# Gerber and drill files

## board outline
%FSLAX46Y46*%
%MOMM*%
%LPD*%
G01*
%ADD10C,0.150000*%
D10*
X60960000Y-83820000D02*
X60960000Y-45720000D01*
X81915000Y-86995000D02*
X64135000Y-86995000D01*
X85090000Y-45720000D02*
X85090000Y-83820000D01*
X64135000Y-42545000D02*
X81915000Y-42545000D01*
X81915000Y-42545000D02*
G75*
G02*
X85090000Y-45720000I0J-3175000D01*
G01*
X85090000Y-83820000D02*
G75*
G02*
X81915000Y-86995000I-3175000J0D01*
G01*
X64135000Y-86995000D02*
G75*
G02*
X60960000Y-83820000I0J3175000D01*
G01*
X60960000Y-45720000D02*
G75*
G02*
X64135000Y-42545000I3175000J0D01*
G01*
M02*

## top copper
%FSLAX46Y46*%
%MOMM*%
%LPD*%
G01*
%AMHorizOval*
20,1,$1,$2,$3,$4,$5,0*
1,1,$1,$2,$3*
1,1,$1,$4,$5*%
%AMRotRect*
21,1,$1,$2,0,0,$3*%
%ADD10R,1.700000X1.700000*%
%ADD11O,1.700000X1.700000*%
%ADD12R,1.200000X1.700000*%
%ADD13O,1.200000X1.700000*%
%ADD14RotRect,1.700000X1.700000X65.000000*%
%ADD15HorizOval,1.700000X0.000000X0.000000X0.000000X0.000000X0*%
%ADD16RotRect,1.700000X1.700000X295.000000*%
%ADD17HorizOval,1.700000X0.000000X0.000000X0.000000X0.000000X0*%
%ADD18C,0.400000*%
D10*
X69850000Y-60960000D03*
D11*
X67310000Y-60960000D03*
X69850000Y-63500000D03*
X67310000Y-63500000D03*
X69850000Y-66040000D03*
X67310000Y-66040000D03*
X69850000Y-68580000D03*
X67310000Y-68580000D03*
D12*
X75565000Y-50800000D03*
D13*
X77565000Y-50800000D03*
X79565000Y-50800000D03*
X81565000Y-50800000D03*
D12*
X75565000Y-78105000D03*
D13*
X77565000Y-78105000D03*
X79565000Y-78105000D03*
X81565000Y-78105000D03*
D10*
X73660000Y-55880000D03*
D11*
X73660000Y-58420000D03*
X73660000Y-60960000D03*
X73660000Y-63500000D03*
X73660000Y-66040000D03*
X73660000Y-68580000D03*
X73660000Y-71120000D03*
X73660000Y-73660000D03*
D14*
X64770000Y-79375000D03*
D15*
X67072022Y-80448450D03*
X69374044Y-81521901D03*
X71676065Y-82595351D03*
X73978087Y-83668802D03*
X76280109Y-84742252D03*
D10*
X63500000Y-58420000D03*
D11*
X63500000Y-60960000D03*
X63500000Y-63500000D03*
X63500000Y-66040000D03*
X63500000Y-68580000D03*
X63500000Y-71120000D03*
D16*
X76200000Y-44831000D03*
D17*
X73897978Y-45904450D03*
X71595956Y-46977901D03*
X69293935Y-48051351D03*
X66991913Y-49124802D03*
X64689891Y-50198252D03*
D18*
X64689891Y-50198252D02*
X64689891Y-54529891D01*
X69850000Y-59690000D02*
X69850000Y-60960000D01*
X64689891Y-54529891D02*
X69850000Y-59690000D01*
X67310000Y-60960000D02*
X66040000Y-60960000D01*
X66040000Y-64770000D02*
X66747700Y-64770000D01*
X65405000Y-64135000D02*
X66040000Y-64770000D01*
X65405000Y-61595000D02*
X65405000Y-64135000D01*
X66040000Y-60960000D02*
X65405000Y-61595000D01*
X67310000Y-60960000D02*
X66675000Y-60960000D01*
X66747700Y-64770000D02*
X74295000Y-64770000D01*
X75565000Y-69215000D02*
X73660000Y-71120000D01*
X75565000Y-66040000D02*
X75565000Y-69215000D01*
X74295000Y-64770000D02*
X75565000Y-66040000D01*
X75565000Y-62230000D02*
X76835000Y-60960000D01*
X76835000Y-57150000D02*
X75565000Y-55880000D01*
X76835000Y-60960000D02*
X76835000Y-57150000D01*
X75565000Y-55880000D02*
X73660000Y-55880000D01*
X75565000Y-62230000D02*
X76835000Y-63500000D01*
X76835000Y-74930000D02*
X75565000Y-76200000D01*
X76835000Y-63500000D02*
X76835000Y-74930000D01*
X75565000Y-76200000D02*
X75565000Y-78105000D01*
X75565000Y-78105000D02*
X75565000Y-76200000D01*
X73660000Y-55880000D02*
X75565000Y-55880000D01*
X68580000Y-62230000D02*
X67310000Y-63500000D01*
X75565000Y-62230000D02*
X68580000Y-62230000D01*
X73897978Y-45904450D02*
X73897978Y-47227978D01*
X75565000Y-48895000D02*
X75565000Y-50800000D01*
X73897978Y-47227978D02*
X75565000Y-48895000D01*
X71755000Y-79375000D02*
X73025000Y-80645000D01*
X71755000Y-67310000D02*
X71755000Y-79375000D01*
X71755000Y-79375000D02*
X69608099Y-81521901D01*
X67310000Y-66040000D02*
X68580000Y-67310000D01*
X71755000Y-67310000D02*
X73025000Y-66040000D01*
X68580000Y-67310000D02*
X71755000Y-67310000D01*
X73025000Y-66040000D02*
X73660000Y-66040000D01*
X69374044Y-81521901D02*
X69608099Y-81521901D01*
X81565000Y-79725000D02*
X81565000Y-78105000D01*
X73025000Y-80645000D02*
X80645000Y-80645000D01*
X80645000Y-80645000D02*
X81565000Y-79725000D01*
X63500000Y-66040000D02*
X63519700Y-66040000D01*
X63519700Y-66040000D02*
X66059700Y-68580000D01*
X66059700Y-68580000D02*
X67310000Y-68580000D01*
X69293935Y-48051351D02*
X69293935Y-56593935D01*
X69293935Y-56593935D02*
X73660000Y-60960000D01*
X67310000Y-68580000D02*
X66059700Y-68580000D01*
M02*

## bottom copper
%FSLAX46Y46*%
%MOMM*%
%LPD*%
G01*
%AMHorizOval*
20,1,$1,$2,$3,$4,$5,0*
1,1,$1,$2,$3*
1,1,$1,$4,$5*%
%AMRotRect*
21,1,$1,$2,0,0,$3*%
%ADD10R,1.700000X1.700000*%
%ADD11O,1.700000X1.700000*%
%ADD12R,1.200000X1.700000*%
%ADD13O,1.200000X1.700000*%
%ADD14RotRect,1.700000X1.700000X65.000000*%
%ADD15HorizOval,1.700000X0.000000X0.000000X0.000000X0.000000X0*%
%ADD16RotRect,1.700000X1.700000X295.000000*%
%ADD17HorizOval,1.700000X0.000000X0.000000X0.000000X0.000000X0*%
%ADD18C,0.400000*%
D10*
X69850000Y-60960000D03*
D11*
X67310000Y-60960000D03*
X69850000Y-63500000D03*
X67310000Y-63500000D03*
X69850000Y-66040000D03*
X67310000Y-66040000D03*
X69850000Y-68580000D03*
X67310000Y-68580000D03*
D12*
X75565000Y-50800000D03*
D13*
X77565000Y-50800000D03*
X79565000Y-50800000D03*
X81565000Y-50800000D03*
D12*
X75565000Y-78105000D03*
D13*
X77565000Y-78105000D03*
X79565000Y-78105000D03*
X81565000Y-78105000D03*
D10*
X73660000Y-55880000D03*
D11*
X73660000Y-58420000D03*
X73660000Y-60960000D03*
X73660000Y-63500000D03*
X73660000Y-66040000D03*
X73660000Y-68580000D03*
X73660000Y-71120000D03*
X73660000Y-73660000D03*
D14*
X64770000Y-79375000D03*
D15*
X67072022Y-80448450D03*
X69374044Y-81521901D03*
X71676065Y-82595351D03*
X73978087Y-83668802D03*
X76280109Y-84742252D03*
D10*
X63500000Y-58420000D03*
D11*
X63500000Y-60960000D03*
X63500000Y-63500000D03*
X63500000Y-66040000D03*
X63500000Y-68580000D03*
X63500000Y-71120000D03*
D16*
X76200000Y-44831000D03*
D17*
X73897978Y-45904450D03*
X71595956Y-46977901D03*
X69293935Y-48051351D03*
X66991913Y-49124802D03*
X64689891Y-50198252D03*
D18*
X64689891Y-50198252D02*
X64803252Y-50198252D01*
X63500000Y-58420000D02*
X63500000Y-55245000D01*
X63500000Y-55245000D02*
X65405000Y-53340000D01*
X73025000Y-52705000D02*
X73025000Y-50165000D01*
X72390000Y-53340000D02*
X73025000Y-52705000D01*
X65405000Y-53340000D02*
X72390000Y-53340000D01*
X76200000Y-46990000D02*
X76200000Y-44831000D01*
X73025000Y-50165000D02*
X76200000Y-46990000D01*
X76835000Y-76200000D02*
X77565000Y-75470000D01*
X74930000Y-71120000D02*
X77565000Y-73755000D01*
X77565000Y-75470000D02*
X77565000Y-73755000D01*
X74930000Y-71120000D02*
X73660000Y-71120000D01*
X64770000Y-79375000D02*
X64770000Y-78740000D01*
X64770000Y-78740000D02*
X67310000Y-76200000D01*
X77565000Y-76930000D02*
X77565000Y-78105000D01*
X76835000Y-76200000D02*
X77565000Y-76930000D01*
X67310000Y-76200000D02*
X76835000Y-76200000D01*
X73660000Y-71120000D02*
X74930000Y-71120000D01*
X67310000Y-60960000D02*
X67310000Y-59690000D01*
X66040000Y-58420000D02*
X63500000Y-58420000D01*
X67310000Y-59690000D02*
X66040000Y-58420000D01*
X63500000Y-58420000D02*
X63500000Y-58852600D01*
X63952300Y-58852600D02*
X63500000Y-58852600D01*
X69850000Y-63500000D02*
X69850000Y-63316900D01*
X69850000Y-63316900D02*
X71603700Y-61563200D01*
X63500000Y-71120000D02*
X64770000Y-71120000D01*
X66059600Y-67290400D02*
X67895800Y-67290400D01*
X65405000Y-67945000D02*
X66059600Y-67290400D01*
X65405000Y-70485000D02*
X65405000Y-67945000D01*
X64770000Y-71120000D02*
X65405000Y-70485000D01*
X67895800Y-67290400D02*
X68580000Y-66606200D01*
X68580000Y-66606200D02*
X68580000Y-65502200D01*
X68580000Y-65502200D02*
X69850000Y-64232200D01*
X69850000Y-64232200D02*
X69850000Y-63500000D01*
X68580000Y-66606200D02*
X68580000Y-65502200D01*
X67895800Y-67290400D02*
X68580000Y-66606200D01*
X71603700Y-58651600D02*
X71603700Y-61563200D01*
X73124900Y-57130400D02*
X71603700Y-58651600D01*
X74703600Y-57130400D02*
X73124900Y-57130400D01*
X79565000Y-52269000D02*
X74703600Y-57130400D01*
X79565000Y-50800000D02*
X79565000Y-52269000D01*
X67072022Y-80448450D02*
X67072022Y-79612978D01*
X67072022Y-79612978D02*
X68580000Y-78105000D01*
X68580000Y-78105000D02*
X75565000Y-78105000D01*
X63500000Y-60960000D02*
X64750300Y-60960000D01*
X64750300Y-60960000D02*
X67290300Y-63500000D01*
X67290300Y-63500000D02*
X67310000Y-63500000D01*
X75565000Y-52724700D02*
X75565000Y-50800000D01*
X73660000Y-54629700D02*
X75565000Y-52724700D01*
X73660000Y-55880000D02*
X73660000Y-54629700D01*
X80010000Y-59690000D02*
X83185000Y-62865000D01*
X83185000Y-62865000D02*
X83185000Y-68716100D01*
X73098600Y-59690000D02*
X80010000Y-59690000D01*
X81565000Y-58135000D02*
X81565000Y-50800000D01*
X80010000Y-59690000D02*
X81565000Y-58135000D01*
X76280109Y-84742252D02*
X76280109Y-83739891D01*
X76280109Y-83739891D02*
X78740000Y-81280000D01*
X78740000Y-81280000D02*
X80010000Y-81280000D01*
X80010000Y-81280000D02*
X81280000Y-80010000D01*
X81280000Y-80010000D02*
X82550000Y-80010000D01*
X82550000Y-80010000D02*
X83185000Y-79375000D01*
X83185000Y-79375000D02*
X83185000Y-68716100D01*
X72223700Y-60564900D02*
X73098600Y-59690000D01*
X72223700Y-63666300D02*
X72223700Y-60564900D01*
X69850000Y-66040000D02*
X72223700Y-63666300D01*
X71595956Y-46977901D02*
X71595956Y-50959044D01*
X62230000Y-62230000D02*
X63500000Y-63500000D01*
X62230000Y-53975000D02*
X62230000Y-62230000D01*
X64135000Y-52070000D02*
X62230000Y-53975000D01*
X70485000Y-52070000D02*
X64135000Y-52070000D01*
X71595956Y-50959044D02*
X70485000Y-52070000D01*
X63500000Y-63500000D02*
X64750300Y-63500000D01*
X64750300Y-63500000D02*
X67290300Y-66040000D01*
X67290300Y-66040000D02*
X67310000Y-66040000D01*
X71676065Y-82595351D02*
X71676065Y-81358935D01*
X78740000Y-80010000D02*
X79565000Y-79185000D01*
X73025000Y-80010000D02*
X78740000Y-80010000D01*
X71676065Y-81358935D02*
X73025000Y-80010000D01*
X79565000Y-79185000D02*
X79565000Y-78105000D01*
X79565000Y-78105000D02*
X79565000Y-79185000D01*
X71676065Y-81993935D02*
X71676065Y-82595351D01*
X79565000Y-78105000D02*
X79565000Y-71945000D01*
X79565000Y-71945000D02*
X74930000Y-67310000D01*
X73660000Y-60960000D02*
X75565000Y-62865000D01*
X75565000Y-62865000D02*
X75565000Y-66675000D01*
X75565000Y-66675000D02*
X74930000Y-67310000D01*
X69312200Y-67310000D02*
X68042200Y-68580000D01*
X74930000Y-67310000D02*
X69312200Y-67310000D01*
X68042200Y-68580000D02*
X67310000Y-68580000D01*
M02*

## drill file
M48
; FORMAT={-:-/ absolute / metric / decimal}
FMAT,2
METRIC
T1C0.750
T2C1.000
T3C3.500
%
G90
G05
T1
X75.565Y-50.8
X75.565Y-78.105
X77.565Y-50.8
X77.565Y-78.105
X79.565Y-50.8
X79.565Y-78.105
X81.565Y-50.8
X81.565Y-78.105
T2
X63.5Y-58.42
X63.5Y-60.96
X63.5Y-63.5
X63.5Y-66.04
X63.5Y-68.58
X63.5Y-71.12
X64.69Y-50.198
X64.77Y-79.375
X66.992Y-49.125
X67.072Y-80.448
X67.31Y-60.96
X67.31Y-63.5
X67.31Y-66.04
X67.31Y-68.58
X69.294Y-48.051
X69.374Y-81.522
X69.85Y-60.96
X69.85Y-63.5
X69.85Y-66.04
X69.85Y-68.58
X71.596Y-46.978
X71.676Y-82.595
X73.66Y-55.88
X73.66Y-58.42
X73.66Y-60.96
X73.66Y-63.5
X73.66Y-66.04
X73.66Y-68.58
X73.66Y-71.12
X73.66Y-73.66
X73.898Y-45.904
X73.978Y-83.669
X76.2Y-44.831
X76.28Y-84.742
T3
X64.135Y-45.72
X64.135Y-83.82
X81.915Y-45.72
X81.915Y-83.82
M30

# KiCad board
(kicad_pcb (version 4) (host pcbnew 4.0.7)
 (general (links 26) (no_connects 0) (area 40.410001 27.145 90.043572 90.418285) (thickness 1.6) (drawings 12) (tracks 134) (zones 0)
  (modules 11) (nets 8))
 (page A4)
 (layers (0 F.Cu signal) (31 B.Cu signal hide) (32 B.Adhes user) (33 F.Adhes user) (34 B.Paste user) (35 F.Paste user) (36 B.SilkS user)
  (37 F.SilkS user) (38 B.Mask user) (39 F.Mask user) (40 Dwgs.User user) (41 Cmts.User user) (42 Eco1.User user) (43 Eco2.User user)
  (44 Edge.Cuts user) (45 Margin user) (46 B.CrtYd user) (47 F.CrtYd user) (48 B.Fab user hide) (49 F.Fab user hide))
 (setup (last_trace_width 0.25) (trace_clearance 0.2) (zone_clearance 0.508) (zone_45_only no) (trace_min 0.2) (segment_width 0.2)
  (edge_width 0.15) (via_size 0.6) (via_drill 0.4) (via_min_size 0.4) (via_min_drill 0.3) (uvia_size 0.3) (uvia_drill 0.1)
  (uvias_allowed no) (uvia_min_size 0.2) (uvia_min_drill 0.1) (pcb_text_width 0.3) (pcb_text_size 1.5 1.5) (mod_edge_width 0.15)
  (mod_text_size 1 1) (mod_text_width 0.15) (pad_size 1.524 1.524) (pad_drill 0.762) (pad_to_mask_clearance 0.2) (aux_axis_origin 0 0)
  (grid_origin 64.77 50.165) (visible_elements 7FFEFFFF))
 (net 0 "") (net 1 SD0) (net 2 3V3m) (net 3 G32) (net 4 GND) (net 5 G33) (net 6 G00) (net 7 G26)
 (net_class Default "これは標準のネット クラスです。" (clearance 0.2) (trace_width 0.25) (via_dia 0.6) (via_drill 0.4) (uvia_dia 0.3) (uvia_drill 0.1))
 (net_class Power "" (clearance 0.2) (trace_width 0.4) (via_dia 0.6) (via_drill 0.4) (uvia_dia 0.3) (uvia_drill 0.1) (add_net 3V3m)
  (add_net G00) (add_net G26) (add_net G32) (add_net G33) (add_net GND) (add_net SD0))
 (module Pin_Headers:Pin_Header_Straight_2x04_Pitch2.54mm (layer B.Cu) (at 69.85 60.96 180)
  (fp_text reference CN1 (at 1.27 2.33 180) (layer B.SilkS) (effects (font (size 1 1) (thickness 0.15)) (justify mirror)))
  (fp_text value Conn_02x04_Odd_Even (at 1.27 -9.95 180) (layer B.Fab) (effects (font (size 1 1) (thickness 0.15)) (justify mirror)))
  (pad 1 thru_hole rect (at 0 0 180) (size 1.7 1.7) (drill 1) (layers *.Cu *.Mask) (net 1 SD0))
  (pad 2 thru_hole oval (at 2.54 0 180) (size 1.7 1.7) (drill 1) (layers *.Cu *.Mask) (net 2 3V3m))
  (pad 3 thru_hole oval (at 0 -2.54 180) (size 1.7 1.7) (drill 1) (layers *.Cu *.Mask) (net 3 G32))
  (pad 4 thru_hole oval (at 2.54 -2.54 180) (size 1.7 1.7) (drill 1) (layers *.Cu *.Mask) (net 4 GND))
  (pad 5 thru_hole oval (at 0 -5.08 180) (size 1.7 1.7) (drill 1) (layers *.Cu *.Mask) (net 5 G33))
  (pad 6 thru_hole oval (at 2.54 -5.08 180) (size 1.7 1.7) (drill 1) (layers *.Cu *.Mask) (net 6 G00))
  (pad 7 thru_hole oval (at 0 -7.62 180) (size 1.7 1.7) (drill 1) (layers *.Cu *.Mask))
  (pad 8 thru_hole oval (at 2.54 -7.62 180) (size 1.7 1.7) (drill 1) (layers *.Cu *.Mask) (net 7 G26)))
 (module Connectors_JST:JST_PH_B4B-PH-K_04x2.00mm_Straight (layer F.Cu) (at 75.565 50.8)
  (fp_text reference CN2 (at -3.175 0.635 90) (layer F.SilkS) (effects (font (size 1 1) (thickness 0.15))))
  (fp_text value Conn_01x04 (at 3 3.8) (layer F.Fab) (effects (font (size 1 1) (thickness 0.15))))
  (pad 1 thru_hole rect (at 0 0) (size 1.2 1.7) (drill 0.75) (layers *.Cu *.Mask) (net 4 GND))
  (pad 2 thru_hole oval (at 2 0) (size 1.2 1.7) (drill 0.75) (layers *.Cu *.Mask))
  (pad 3 thru_hole oval (at 4 0) (size 1.2 1.7) (drill 0.75) (layers *.Cu *.Mask) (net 3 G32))
  (pad 4 thru_hole oval (at 6 0) (size 1.2 1.7) (drill 0.75) (layers *.Cu *.Mask) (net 5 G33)))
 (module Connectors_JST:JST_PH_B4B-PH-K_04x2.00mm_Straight (layer F.Cu) (at 75.565 78.105)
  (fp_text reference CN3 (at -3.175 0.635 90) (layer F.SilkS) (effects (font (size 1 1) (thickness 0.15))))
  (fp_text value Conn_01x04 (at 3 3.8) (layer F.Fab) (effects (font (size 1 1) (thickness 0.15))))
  (pad 1 thru_hole rect (at 0 0) (size 1.2 1.7) (drill 0.75) (layers *.Cu *.Mask) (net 4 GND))
  (pad 2 thru_hole oval (at 2 0) (size 1.2 1.7) (drill 0.75) (layers *.Cu *.Mask) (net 2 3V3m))
  (pad 3 thru_hole oval (at 4 0) (size 1.2 1.7) (drill 0.75) (layers *.Cu *.Mask) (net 7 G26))
  (pad 4 thru_hole oval (at 6 0) (size 1.2 1.7) (drill 0.75) (layers *.Cu *.Mask) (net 6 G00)))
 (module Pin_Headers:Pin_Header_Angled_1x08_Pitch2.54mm (layer F.Cu) (at 73.66 55.88)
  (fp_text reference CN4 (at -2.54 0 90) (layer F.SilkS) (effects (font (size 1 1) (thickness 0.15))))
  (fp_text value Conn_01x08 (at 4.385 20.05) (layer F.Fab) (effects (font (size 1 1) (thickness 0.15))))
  (pad 1 thru_hole rect (at 0 0) (size 1.7 1.7) (drill 1) (layers *.Cu *.Mask) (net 4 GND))
  (pad 2 thru_hole oval (at 0 2.54) (size 1.7 1.7) (drill 1) (layers *.Cu *.Mask))
  (pad 3 thru_hole oval (at 0 5.08) (size 1.7 1.7) (drill 1) (layers *.Cu *.Mask) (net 7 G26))
  (pad 4 thru_hole oval (at 0 7.62) (size 1.7 1.7) (drill 1) (layers *.Cu *.Mask))
  (pad 5 thru_hole oval (at 0 10.16) (size 1.7 1.7) (drill 1) (layers *.Cu *.Mask) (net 6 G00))
  (pad 6 thru_hole oval (at 0 12.7) (size 1.7 1.7) (drill 1) (layers *.Cu *.Mask))
  (pad 7 thru_hole oval (at 0 15.24) (size 1.7 1.7) (drill 1) (layers *.Cu *.Mask) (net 2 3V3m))
  (pad 8 thru_hole oval (at 0 17.78) (size 1.7 1.7) (drill 1) (layers *.Cu *.Mask)))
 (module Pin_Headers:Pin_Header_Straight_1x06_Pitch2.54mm (layer F.Cu) (at 64.77 79.375 65)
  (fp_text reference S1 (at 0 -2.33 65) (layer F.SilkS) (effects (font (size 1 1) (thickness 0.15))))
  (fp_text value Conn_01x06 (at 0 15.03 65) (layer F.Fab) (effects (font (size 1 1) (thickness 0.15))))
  (pad 1 thru_hole rect (at 0 0 65) (size 1.7 1.7) (drill 1) (layers *.Cu *.Mask) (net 2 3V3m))
  (pad 2 thru_hole oval (at 0 2.54 65) (size 1.7 1.7) (drill 1) (layers *.Cu *.Mask) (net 4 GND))
  (pad 3 thru_hole oval (at 0 5.08 65) (size 1.7 1.7) (drill 1) (layers *.Cu *.Mask) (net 6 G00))
  (pad 4 thru_hole oval (at 0 7.62 65) (size 1.7 1.7) (drill 1) (layers *.Cu *.Mask) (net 7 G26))
  (pad 5 thru_hole oval (at 0 10.16 65) (size 1.7 1.7) (drill 1) (layers *.Cu *.Mask))
  (pad 6 thru_hole oval (at 0 12.7 65) (size 1.7 1.7) (drill 1) (layers *.Cu *.Mask) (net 5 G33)))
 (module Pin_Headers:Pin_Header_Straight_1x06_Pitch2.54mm (layer F.Cu) (at 63.5 58.42)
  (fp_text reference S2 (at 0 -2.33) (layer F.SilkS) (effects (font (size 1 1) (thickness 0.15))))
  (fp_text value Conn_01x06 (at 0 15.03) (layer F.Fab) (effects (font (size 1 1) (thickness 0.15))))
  (pad 1 thru_hole rect (at 0 0) (size 1.7 1.7) (drill 1) (layers *.Cu *.Mask) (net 2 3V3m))
  (pad 2 thru_hole oval (at 0 2.54) (size 1.7 1.7) (drill 1) (layers *.Cu *.Mask) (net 4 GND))
  (pad 3 thru_hole oval (at 0 5.08) (size 1.7 1.7) (drill 1) (layers *.Cu *.Mask) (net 6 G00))
  (pad 4 thru_hole oval (at 0 7.62) (size 1.7 1.7) (drill 1) (layers *.Cu *.Mask) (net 7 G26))
  (pad 5 thru_hole oval (at 0 10.16) (size 1.7 1.7) (drill 1) (layers *.Cu *.Mask))
  (pad 6 thru_hole oval (at 0 12.7) (size 1.7 1.7) (drill 1) (layers *.Cu *.Mask) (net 3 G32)))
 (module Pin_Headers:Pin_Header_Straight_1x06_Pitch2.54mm (layer F.Cu) (at 76.2 44.831 295)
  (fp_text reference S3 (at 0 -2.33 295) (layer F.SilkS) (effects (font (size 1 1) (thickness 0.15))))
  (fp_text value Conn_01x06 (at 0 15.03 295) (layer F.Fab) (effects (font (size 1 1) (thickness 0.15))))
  (pad 1 thru_hole rect (at 0 0 295) (size 1.7 1.7) (drill 1) (layers *.Cu *.Mask) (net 2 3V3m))
  (pad 2 thru_hole oval (at 0 2.54 295) (size 1.7 1.7) (drill 1) (layers *.Cu *.Mask) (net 4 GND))
  (pad 3 thru_hole oval (at 0 5.08 295) (size 1.7 1.7) (drill 1) (layers *.Cu *.Mask) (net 6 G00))
  (pad 4 thru_hole oval (at 0 7.62 295) (size 1.7 1.7) (drill 1) (layers *.Cu *.Mask) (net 7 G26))
  (pad 5 thru_hole oval (at 0 10.16 295) (size 1.7 1.7) (drill 1) (layers *.Cu *.Mask))
  (pad 6 thru_hole oval (at 0 12.7 295) (size 1.7 1.7) (drill 1) (layers *.Cu *.Mask) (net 1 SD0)))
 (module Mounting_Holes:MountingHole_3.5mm (layer F.Cu) (at 64.135 45.72)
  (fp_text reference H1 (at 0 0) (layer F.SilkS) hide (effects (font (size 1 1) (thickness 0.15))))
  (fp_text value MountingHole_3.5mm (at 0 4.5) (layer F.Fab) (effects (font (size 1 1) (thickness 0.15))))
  (pad 1 np_thru_hole circle (at 0 0) (size 3.5 3.5) (drill 3.5) (layers *.Cu *.Mask)))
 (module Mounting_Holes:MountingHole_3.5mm (layer F.Cu) (at 81.915 45.72)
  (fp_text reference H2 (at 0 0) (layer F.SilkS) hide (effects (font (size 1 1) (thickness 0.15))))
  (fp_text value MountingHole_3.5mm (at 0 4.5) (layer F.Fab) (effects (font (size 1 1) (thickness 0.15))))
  (pad 1 np_thru_hole circle (at 0 0) (size 3.5 3.5) (drill 3.5) (layers *.Cu *.Mask)))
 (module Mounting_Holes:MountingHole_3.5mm (layer F.Cu) (at 64.135 83.82)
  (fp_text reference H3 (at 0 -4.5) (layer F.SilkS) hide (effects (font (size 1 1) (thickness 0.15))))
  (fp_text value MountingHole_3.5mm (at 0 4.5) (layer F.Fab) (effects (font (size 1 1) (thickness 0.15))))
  (pad 1 np_thru_hole circle (at 0 0) (size 3.5 3.5) (drill 3.5) (layers *.Cu *.Mask)))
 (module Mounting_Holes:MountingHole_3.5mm (layer F.Cu) (at 81.915 83.82)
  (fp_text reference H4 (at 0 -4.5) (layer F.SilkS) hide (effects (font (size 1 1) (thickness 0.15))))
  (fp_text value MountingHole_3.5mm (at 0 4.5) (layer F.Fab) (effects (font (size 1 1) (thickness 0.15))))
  (pad 1 np_thru_hole circle (at 0 0) (size 3.5 3.5) (drill 3.5) (layers *.Cu *.Mask)))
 (gr_line (start 60.96 83.82) (end 60.96 45.72) (angle 90) (layer Edge.Cuts) (width 0.15))
 (gr_line (start 81.915 86.995) (end 64.135 86.995) (angle 90) (layer Edge.Cuts) (width 0.15))
 (gr_line (start 85.09 45.72) (end 85.09 83.82) (angle 90) (layer Edge.Cuts) (width 0.15))
 (gr_line (start 64.135 42.545) (end 81.915 42.545) (angle 90) (layer Edge.Cuts) (width 0.15))
 (gr_arc (start 81.915 45.72) (end 81.915 42.545) (angle 90) (layer Edge.Cuts) (width 0.15))
 (gr_arc (start 81.915 83.82) (end 85.09 83.82) (angle 90) (layer Edge.Cuts) (width 0.15))
 (gr_arc (start 64.135 83.82) (end 64.135 86.995) (angle 90) (layer Edge.Cuts) (width 0.15))
 (gr_arc (start 64.135 45.72) (end 60.96 45.72) (angle 90) (layer Edge.Cuts) (width 0.15))
 (segment (start 64.689891 50.198252) (end 64.689891 54.529891) (width 0.4) (layer F.Cu) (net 1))
 (segment (start 69.85 59.69) (end 69.85 60.96) (width 0.4) (layer F.Cu) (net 1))
 (segment (start 64.689891 54.529891) (end 69.85 59.69) (width 0.4) (layer F.Cu) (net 1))
 (segment (start 64.689891 50.198252) (end 64.803252 50.198252) (width 0.4) (layer B.Cu) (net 1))
 (segment (start 63.5 58.42) (end 63.5 55.245) (width 0.4) (layer B.Cu) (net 2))
 (segment (start 63.5 55.245) (end 65.405 53.34) (width 0.4) (layer B.Cu) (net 2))
 (segment (start 73.025 52.705) (end 73.025 50.165) (width 0.4) (layer B.Cu) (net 2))
 (segment (start 72.39 53.34) (end 73.025 52.705) (width 0.4) (layer B.Cu) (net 2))
 (segment (start 65.405 53.34) (end 72.39 53.34) (width 0.4) (layer B.Cu) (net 2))
 (segment (start 76.2 46.99) (end 76.2 44.831) (width 0.4) (layer B.Cu) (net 2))
 (segment (start 73.025 50.165) (end 76.2 46.99) (width 0.4) (layer B.Cu) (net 2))
 (segment (start 67.31 60.96) (end 66.04 60.96) (width 0.4) (layer F.Cu) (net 2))
 (segment (start 66.04 64.77) (end 66.7477 64.77) (width 0.4) (layer F.Cu) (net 2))
 (segment (start 65.405 64.135) (end 66.04 64.77) (width 0.4) (layer F.Cu) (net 2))
 (segment (start 65.405 61.595) (end 65.405 64.135) (width 0.4) (layer F.Cu) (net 2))
 (segment (start 66.04 60.96) (end 65.405 61.595) (width 0.4) (layer F.Cu) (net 2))
 (segment (start 67.31 60.96) (end 66.675 60.96) (width 0.4) (layer F.Cu) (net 2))
 (segment (start 66.7477 64.77) (end 74.295 64.77) (width 0.4) (layer F.Cu) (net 2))
 (segment (start 75.565 69.215) (end 73.66 71.12) (width 0.4) (layer F.Cu) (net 2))
 (segment (start 75.565 66.04) (end 75.565 69.215) (width 0.4) (layer F.Cu) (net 2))
 (segment (start 74.295 64.77) (end 75.565 66.04) (width 0.4) (layer F.Cu) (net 2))
 (segment (start 76.835 76.2) (end 77.565 75.47) (width 0.4) (layer B.Cu) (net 2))
 (segment (start 74.93 71.12) (end 77.565 73.755) (width 0.4) (layer B.Cu) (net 2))
 (segment (start 77.565 75.47) (end 77.565 73.755) (width 0.4) (layer B.Cu) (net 2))
 (segment (start 74.93 71.12) (end 73.66 71.12) (width 0.4) (layer B.Cu) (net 2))
 (segment (start 64.77 79.375) (end 64.77 78.74) (width 0.4) (layer B.Cu) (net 2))
 (segment (start 64.77 78.74) (end 67.31 76.2) (width 0.4) (layer B.Cu) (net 2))
 (segment (start 77.565 76.93) (end 77.565 78.105) (width 0.4) (layer B.Cu) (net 2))
 (segment (start 76.835 76.2) (end 77.565 76.93) (width 0.4) (layer B.Cu) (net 2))
 (segment (start 67.31 76.2) (end 76.835 76.2) (width 0.4) (layer B.Cu) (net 2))
 (segment (start 73.66 71.12) (end 74.93 71.12) (width 0.4) (layer B.Cu) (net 2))
 (segment (start 67.31 60.96) (end 67.31 59.69) (width 0.4) (layer B.Cu) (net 2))
 (segment (start 66.04 58.42) (end 63.5 58.42) (width 0.4) (layer B.Cu) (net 2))
 (segment (start 67.31 59.69) (end 66.04 58.42) (width 0.4) (layer B.Cu) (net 2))
 (segment (start 63.5 58.42) (end 63.5 58.8526) (width 0.4) (layer B.Cu) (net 2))
 (segment (start 63.9523 58.8526) (end 63.5 58.8526) (width 0.4) (layer B.Cu) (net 2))
 (segment (start 69.85 63.5) (end 69.85 63.3169) (width 0.4) (layer B.Cu) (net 3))
 (segment (start 69.85 63.3169) (end 71.6037 61.5632) (width 0.4) (layer B.Cu) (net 3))
 (segment (start 63.5 71.12) (end 64.77 71.12) (width 0.4) (layer B.Cu) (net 3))
 (segment (start 66.0596 67.2904) (end 67.8958 67.2904) (width 0.4) (layer B.Cu) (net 3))
 (segment (start 65.405 67.945) (end 66.0596 67.2904) (width 0.4) (layer B.Cu) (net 3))
 (segment (start 65.405 70.485) (end 65.405 67.945) (width 0.4) (layer B.Cu) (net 3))
 (segment (start 64.77 71.12) (end 65.405 70.485) (width 0.4) (layer B.Cu) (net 3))
 (segment (start 67.8958 67.2904) (end 68.58 66.6062) (width 0.4) (layer B.Cu) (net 3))
 (segment (start 68.58 66.6062) (end 68.58 65.5022) (width 0.4) (layer B.Cu) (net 3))
 (segment (start 68.58 65.5022) (end 69.85 64.2322) (width 0.4) (layer B.Cu) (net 3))
 (segment (start 69.85 64.2322) (end 69.85 63.5) (width 0.4) (layer B.Cu) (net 3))
 (segment (start 68.58 66.6062) (end 68.58 65.5022) (width 0.4) (layer B.Cu) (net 3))
 (segment (start 67.8958 67.2904) (end 68.58 66.6062) (width 0.4) (layer B.Cu) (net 3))
 (segment (start 71.6037 58.6516) (end 71.6037 61.5632) (width 0.4) (layer B.Cu) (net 3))
 (segment (start 73.1249 57.1304) (end 71.6037 58.6516) (width 0.4) (layer B.Cu) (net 3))
 (segment (start 74.7036 57.1304) (end 73.1249 57.1304) (width 0.4) (layer B.Cu) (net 3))
 (segment (start 79.565 52.269) (end 74.7036 57.1304) (width 0.4) (layer B.Cu) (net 3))
 (segment (start 79.565 50.8) (end 79.565 52.269) (width 0.4) (layer B.Cu) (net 3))
 (segment (start 75.565 62.23) (end 76.835 60.96) (width 0.4) (layer F.Cu) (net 4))
 (segment (start 76.835 57.15) (end 75.565 55.88) (width 0.4) (layer F.Cu) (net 4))
 (segment (start 76.835 60.96) (end 76.835 57.15) (width 0.4) (layer F.Cu) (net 4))
 (segment (start 75.565 55.88) (end 73.66 55.88) (width 0.4) (layer F.Cu) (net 4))
 (segment (start 75.565 62.23) (end 76.835 63.5) (width 0.4) (layer F.Cu) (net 4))
 (segment (start 76.835 74.93) (end 75.565 76.2) (width 0.4) (layer F.Cu) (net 4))
 (segment (start 76.835 63.5) (end 76.835 74.93) (width 0.4) (layer F.Cu) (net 4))
 (segment (start 75.565 76.2) (end 75.565 78.105) (width 0.4) (layer F.Cu) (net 4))
 (segment (start 75.565 78.105) (end 75.565 76.2) (width 0.4) (layer F.Cu) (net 4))
 (segment (start 73.66 55.88) (end 75.565 55.88) (width 0.4) (layer F.Cu) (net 4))
 (segment (start 68.58 62.23) (end 67.31 63.5) (width 0.4) (layer F.Cu) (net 4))
 (segment (start 75.565 62.23) (end 68.58 62.23) (width 0.4) (layer F.Cu) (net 4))
 (segment (start 67.072022 80.44845) (end 67.072022 79.612978) (width 0.4) (layer B.Cu) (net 4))
 (segment (start 67.072022 79.612978) (end 68.58 78.105) (width 0.4) (layer B.Cu) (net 4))
 (segment (start 68.58 78.105) (end 75.565 78.105) (width 0.4) (layer B.Cu) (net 4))
 (segment (start 63.5 60.96) (end 64.7503 60.96) (width 0.4) (layer B.Cu) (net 4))
 (segment (start 64.7503 60.96) (end 67.2903 63.5) (width 0.4) (layer B.Cu) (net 4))
 (segment (start 67.2903 63.5) (end 67.31 63.5) (width 0.4) (layer B.Cu) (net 4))
 (segment (start 73.897978 45.90445) (end 73.897978 47.227978) (width 0.4) (layer F.Cu) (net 4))
 (segment (start 75.565 48.895) (end 75.565 50.8) (width 0.4) (layer F.Cu) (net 4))
 (segment (start 73.897978 47.227978) (end 75.565 48.895) (width 0.4) (layer F.Cu) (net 4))
 (segment (start 75.565 52.7247) (end 75.565 50.8) (width 0.4) (layer B.Cu) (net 4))
 (segment (start 73.66 54.6297) (end 75.565 52.7247) (width 0.4) (layer B.Cu) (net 4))
 (segment (start 73.66 55.88) (end 73.66 54.6297) (width 0.4) (layer B.Cu) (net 4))
 (segment (start 80.01 59.69) (end 83.185 62.865) (width 0.4) (layer B.Cu) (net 5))
 (segment (start 83.185 62.865) (end 83.185 68.7161) (width 0.4) (layer B.Cu) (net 5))
 (segment (start 73.0986 59.69) (end 80.01 59.69) (width 0.4) (layer B.Cu) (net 5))
 (segment (start 81.565 58.135) (end 81.565 50.8) (width 0.4) (layer B.Cu) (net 5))
 (segment (start 80.01 59.69) (end 81.565 58.135) (width 0.4) (layer B.Cu) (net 5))
 (segment (start 76.280109 84.742252) (end 76.280109 83.739891) (width 0.4) (layer B.Cu) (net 5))
 (segment (start 76.280109 83.739891) (end 78.74 81.28) (width 0.4) (layer B.Cu) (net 5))
 (segment (start 78.74 81.28) (end 80.01 81.28) (width 0.4) (layer B.Cu) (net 5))
 (segment (start 80.01 81.28) (end 81.28 80.01) (width 0.4) (layer B.Cu) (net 5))
 (segment (start 81.28 80.01) (end 82.55 80.01) (width 0.4) (layer B.Cu) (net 5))
 (segment (start 82.55 80.01) (end 83.185 79.375) (width 0.4) (layer B.Cu) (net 5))
 (segment (start 83.185 79.375) (end 83.185 68.7161) (width 0.4) (layer B.Cu) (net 5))
 (segment (start 72.2237 60.5649) (end 73.0986 59.69) (width 0.4) (layer B.Cu) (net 5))
 (segment (start 72.2237 63.6663) (end 72.2237 60.5649) (width 0.4) (layer B.Cu) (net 5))
 (segment (start 69.85 66.04) (end 72.2237 63.6663) (width 0.4) (layer B.Cu) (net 5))
 (segment (start 71.595956 46.977901) (end 71.595956 50.959044) (width 0.4) (layer B.Cu) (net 6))
 (segment (start 62.23 62.23) (end 63.5 63.5) (width 0.4) (layer B.Cu) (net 6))
 (segment (start 62.23 53.975) (end 62.23 62.23) (width 0.4) (layer B.Cu) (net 6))
 (segment (start 64.135 52.07) (end 62.23 53.975) (width 0.4) (layer B.Cu) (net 6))
 (segment (start 70.485 52.07) (end 64.135 52.07) (width 0.4) (layer B.Cu) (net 6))
 (segment (start 71.595956 50.959044) (end 70.485 52.07) (width 0.4) (layer B.Cu) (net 6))
 (segment (start 71.755 79.375) (end 73.025 80.645) (width 0.4) (layer F.Cu) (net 6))
 (segment (start 71.755 67.31) (end 71.755 79.375) (width 0.4) (layer F.Cu) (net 6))
 (segment (start 71.755 79.375) (end 69.608099 81.521901) (width 0.4) (layer F.Cu) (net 6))
 (segment (start 67.31 66.04) (end 68.58 67.31) (width 0.4) (layer F.Cu) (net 6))
 (segment (start 71.755 67.31) (end 73.025 66.04) (width 0.4) (layer F.Cu) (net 6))
 (segment (start 68.58 67.31) (end 71.755 67.31) (width 0.4) (layer F.Cu) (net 6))
 (segment (start 73.025 66.04) (end 73.66 66.04) (width 0.4) (layer F.Cu) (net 6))
 (segment (start 69.374044 81.521901) (end 69.608099 81.521901) (width 0.4) (layer F.Cu) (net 6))
 (segment (start 81.565 79.725) (end 81.565 78.105) (width 0.4) (layer F.Cu) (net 6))
 (segment (start 73.025 80.645) (end 80.645 80.645) (width 0.4) (layer F.Cu) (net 6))
 (segment (start 80.645 80.645) (end 81.565 79.725) (width 0.4) (layer F.Cu) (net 6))
 (segment (start 63.5 63.5) (end 64.7503 63.5) (width 0.4) (layer B.Cu) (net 6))
 (segment (start 64.7503 63.5) (end 67.2903 66.04) (width 0.4) (layer B.Cu) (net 6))
 (segment (start 67.2903 66.04) (end 67.31 66.04) (width 0.4) (layer B.Cu) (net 6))
 (segment (start 71.676065 82.595351) (end 71.676065 81.358935) (width 0.4) (layer B.Cu) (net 7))
 (segment (start 78.74 80.01) (end 79.565 79.185) (width 0.4) (layer B.Cu) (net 7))
 (segment (start 73.025 80.01) (end 78.74 80.01) (width 0.4) (layer B.Cu) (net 7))
 (segment (start 71.676065 81.358935) (end 73.025 80.01) (width 0.4) (layer B.Cu) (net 7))
 (segment (start 79.565 79.185) (end 79.565 78.105) (width 0.4) (layer B.Cu) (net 7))
 (segment (start 63.5 66.04) (end 63.5197 66.04) (width 0.4) (layer F.Cu) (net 7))
 (segment (start 63.5197 66.04) (end 66.0597 68.58) (width 0.4) (layer F.Cu) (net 7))
 (segment (start 66.0597 68.58) (end 67.31 68.58) (width 0.4) (layer F.Cu) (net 7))
 (segment (start 79.565 78.105) (end 79.565 79.185) (width 0.4) (layer B.Cu) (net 7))
 (segment (start 71.676065 81.993935) (end 71.676065 82.595351) (width 0.4) (layer B.Cu) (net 7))
 (segment (start 79.565 78.105) (end 79.565 71.945) (width 0.4) (layer B.Cu) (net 7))
 (segment (start 79.565 71.945) (end 74.93 67.31) (width 0.4) (layer B.Cu) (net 7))
 (segment (start 73.66 60.96) (end 75.565 62.865) (width 0.4) (layer B.Cu) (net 7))
 (segment (start 75.565 62.865) (end 75.565 66.675) (width 0.4) (layer B.Cu) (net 7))
 (segment (start 75.565 66.675) (end 74.93 67.31) (width 0.4) (layer B.Cu) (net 7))
 (segment (start 69.3122 67.31) (end 68.0422 68.58) (width 0.4) (layer B.Cu) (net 7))
 (segment (start 74.93 67.31) (end 69.3122 67.31) (width 0.4) (layer B.Cu) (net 7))
 (segment (start 68.0422 68.58) (end 67.31 68.58) (width 0.4) (layer B.Cu) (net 7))
 (segment (start 69.293935 48.051351) (end 69.293935 56.593935) (width 0.4) (layer F.Cu) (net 7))
 (segment (start 69.293935 56.593935) (end 73.66 60.96) (width 0.4) (layer F.Cu) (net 7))
 (segment (start 67.31 68.58) (end 66.0597 68.58) (width 0.4) (layer F.Cu) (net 7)))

